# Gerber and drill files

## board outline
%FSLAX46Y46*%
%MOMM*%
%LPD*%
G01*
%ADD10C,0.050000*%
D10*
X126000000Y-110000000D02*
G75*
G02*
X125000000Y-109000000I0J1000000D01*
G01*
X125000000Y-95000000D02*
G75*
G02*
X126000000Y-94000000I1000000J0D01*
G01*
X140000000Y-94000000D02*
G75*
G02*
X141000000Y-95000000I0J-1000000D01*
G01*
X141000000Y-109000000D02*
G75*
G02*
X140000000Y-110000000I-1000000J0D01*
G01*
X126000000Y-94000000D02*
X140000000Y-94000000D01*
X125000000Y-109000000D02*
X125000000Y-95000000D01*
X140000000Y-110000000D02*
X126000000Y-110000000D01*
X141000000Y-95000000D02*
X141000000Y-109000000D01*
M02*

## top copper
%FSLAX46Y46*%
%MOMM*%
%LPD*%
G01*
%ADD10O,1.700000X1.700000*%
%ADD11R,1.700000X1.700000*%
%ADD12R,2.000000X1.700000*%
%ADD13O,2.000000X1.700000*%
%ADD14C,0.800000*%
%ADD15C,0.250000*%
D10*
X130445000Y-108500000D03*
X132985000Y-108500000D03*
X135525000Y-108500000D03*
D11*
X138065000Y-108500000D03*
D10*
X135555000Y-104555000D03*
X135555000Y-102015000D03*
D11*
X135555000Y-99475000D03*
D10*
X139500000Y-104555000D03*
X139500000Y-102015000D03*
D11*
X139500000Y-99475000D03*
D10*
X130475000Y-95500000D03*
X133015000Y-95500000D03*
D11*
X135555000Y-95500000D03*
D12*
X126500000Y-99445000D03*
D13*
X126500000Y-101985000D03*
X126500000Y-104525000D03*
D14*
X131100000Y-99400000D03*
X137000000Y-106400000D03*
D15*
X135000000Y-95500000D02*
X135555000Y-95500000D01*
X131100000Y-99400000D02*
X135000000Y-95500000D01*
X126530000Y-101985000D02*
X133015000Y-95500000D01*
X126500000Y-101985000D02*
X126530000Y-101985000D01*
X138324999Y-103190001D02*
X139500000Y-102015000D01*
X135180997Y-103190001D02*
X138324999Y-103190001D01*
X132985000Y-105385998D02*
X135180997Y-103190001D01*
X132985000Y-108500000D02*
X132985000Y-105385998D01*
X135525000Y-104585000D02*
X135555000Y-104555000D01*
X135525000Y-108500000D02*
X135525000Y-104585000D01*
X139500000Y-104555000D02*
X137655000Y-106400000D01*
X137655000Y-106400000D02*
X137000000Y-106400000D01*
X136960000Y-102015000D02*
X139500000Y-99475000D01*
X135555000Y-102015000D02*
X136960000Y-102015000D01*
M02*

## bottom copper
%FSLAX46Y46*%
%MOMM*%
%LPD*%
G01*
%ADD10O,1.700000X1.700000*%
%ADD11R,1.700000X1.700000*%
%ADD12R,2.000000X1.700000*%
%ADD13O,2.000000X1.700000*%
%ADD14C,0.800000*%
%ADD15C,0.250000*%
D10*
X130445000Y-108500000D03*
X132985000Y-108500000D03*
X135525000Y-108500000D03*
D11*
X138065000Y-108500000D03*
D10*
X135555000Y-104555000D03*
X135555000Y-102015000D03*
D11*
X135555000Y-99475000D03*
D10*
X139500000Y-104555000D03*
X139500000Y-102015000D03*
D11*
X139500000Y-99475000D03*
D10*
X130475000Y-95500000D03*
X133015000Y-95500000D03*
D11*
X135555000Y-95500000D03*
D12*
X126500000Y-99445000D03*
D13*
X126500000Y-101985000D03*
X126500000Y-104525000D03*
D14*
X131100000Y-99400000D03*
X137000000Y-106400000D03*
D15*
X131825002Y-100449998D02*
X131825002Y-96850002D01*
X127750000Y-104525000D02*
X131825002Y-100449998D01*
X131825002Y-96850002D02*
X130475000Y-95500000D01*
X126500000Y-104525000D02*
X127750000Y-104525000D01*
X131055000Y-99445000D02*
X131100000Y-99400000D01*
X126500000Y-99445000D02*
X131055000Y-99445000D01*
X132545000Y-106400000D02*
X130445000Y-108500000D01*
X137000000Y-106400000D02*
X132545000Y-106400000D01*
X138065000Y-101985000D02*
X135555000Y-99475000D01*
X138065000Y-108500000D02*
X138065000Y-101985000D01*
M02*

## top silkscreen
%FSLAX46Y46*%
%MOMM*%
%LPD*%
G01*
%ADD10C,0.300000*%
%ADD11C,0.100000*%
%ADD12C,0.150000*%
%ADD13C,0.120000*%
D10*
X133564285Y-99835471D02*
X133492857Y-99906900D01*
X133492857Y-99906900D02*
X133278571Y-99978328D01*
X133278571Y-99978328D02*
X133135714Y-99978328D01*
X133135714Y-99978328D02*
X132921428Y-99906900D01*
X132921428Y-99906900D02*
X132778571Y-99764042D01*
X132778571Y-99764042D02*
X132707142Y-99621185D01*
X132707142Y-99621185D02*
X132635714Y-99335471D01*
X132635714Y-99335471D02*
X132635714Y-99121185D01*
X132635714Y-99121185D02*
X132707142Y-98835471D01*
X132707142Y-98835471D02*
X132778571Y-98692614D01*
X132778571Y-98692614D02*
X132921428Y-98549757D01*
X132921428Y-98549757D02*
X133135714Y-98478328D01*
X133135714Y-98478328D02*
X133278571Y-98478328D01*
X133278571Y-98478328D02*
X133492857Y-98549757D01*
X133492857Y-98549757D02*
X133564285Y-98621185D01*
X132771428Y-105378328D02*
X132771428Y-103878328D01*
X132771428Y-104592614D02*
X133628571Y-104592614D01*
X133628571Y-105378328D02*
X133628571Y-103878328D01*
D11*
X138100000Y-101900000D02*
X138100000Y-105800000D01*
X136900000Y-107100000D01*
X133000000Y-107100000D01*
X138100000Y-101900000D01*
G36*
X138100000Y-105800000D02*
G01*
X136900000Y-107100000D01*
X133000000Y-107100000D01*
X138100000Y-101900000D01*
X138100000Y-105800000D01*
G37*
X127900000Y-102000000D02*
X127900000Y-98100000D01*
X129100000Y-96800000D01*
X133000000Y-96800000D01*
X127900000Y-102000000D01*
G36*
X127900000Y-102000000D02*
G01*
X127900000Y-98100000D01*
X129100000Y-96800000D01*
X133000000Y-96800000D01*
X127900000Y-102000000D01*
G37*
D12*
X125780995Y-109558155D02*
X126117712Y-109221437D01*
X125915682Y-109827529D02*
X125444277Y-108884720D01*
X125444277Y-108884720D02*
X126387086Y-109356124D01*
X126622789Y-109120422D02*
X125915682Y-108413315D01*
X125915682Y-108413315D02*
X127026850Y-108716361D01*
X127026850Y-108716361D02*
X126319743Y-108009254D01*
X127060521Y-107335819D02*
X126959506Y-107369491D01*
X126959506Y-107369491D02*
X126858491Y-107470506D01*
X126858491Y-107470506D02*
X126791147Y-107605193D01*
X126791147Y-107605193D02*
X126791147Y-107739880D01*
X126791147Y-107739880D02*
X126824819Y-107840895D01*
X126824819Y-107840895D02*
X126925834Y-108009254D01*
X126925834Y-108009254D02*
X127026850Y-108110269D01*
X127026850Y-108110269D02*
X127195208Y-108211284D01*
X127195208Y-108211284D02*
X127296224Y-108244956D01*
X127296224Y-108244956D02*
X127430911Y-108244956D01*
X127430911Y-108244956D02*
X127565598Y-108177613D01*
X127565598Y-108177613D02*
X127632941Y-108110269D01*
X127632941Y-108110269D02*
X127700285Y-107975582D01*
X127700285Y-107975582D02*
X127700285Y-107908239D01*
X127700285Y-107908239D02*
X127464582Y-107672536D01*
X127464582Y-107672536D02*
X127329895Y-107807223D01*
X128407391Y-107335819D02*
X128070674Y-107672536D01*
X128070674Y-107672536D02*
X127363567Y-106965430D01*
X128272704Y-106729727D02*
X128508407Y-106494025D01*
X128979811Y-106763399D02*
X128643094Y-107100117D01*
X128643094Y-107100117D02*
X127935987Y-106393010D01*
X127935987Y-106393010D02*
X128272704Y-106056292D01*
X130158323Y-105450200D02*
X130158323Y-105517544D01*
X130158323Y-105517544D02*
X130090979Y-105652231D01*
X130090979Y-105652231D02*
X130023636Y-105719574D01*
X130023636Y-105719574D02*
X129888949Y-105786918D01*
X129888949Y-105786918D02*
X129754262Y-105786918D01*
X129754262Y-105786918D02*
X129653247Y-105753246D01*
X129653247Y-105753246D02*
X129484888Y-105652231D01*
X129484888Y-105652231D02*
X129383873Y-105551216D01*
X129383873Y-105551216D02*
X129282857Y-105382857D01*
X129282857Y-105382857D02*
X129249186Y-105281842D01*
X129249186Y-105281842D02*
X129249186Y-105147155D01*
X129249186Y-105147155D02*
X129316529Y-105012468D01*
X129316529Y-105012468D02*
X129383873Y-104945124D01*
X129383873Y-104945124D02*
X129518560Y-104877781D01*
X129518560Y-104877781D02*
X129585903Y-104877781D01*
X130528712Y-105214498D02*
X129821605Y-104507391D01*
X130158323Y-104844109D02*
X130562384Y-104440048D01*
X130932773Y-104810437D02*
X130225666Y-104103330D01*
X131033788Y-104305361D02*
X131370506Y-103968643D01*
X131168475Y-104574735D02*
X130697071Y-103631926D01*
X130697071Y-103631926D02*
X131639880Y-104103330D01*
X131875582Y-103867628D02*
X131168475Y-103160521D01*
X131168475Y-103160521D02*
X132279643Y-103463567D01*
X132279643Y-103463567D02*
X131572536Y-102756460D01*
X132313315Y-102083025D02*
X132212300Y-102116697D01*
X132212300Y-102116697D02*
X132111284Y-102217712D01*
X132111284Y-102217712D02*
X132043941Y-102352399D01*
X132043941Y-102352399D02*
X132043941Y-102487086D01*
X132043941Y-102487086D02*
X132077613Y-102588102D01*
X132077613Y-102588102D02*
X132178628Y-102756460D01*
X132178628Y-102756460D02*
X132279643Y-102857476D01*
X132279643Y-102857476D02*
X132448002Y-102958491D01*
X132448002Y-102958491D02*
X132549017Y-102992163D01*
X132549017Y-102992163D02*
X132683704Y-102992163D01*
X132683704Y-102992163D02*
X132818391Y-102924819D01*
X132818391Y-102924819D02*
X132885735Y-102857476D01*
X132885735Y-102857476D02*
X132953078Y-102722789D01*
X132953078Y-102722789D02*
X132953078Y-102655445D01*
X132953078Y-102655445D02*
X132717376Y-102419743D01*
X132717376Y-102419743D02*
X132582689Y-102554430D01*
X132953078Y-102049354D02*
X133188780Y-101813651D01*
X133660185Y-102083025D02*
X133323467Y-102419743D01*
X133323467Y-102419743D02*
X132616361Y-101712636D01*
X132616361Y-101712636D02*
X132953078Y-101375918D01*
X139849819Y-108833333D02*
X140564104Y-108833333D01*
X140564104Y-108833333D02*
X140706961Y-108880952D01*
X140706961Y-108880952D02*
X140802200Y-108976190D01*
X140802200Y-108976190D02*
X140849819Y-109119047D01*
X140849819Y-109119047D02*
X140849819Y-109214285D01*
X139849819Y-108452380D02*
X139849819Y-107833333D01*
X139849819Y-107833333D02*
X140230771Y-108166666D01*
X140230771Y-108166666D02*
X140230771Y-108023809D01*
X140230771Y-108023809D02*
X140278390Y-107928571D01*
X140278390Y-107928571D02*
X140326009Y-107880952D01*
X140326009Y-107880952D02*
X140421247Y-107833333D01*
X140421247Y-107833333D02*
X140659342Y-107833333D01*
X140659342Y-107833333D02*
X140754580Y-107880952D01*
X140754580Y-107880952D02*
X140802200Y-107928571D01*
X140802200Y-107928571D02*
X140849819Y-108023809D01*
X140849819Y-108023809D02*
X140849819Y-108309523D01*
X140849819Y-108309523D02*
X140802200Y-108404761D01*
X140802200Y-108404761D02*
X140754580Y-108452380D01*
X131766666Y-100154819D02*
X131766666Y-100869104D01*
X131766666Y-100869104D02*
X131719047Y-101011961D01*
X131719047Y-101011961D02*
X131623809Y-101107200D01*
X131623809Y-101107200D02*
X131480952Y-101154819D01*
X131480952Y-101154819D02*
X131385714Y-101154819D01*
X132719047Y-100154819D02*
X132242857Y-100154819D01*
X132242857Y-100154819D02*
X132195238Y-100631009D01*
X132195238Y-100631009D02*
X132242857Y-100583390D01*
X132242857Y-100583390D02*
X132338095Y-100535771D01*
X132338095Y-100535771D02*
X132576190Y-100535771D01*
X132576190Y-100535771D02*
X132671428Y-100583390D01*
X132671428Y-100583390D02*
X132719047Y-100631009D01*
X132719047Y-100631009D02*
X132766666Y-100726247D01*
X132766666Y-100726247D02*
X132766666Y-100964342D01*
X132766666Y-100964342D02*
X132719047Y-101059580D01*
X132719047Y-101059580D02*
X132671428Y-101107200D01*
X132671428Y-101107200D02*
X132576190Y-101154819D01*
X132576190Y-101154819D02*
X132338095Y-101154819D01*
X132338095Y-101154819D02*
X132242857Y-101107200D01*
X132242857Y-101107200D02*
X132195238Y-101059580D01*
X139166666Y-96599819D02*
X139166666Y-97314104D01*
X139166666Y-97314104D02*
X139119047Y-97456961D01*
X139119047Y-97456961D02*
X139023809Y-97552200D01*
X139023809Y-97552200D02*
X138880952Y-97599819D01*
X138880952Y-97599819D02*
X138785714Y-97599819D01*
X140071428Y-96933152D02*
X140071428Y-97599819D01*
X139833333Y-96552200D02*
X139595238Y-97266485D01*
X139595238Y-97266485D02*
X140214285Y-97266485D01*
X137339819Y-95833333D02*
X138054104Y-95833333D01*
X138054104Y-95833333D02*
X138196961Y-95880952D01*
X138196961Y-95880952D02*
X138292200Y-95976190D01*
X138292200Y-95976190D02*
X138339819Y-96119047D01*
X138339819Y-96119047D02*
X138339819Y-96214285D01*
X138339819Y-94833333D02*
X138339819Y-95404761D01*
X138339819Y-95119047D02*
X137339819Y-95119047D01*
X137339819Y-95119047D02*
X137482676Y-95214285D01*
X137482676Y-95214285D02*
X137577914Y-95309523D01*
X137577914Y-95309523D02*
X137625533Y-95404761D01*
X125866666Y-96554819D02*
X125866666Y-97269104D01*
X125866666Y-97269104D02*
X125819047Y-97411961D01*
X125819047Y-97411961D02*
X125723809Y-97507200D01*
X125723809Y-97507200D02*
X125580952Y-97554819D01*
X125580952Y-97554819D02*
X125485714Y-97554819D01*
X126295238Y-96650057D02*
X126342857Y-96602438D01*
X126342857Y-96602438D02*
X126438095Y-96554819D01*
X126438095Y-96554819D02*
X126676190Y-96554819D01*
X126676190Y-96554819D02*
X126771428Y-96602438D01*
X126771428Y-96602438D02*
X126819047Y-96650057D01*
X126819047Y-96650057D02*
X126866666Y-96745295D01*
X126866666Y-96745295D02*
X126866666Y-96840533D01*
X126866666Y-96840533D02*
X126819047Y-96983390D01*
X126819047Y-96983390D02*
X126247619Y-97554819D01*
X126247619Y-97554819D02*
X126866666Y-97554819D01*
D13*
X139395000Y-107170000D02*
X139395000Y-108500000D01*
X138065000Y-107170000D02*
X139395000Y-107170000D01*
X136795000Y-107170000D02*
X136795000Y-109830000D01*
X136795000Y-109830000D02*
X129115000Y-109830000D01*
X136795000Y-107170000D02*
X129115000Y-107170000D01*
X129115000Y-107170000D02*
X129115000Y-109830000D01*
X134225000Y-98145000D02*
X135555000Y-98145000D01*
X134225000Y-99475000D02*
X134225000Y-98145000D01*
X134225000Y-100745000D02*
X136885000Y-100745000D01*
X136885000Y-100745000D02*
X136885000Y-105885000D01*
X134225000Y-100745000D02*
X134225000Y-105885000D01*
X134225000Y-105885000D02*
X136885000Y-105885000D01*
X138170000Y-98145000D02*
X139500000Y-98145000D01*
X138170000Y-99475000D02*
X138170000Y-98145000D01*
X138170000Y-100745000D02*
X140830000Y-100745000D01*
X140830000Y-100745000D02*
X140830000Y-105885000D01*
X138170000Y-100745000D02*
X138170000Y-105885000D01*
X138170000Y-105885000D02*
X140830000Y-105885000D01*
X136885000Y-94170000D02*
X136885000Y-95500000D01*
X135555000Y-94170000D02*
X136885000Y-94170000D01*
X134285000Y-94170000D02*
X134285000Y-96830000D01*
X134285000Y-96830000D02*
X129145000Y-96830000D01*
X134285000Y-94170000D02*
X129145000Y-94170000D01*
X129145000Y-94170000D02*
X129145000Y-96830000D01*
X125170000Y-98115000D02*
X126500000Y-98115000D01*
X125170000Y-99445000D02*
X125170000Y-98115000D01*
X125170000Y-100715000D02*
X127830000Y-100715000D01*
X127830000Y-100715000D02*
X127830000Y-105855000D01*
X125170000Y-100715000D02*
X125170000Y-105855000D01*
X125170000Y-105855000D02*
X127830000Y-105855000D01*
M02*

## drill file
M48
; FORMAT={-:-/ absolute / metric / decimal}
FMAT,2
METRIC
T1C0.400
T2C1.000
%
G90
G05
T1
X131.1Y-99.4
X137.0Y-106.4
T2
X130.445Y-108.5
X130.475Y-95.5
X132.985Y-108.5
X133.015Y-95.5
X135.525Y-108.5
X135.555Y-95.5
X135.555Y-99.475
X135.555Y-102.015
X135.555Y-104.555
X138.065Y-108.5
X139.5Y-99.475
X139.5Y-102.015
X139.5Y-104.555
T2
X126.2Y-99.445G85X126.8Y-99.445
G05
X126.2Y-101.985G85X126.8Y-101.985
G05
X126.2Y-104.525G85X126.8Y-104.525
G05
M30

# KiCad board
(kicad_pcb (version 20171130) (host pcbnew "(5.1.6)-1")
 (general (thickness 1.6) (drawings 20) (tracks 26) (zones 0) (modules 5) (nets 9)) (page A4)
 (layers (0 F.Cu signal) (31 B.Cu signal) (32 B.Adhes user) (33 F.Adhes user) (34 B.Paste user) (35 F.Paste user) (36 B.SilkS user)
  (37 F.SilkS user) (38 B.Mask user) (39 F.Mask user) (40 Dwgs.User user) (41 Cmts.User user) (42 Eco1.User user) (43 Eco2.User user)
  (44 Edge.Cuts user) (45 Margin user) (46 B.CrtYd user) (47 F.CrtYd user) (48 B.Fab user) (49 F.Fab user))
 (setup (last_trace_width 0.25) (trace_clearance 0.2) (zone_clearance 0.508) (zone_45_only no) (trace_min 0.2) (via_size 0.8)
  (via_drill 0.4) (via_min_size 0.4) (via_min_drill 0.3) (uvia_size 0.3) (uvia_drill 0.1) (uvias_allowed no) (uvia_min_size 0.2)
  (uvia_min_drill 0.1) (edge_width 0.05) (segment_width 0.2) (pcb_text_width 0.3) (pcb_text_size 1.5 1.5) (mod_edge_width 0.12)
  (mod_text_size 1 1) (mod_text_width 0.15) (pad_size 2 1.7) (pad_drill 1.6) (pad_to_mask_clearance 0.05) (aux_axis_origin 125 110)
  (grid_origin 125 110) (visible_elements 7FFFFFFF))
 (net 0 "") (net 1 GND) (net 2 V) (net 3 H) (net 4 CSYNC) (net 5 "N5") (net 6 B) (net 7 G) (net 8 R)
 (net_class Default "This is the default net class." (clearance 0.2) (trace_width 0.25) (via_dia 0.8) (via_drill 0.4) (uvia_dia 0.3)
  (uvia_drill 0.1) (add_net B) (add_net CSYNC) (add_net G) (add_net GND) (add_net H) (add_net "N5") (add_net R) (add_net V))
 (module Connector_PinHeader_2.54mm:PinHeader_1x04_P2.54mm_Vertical (layer F.Cu) (at 138.065 108.5 270)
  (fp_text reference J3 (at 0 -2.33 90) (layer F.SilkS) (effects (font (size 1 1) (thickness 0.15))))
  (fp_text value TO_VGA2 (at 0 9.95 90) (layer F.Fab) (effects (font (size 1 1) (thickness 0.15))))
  (fp_line (start -1.33 -1.33) (end 0 -1.33) (layer F.SilkS) (width 0.12))
  (fp_line (start -1.33 0) (end -1.33 -1.33) (layer F.SilkS) (width 0.12))
  (fp_line (start -1.33 1.27) (end 1.33 1.27) (layer F.SilkS) (width 0.12))
  (fp_line (start 1.33 1.27) (end 1.33 8.95) (layer F.SilkS) (width 0.12))
  (fp_line (start -1.33 1.27) (end -1.33 8.95) (layer F.SilkS) (width 0.12))
  (fp_line (start -1.33 8.95) (end 1.33 8.95) (layer F.SilkS) (width 0.12))
  (pad 4 thru_hole oval (at 0 7.62 270) (size 1.7 1.7) (drill 1) (layers *.Cu *.Mask) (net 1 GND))
  (pad 3 thru_hole oval (at 0 5.08 270) (size 1.7 1.7) (drill 1) (layers *.Cu *.Mask) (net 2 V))
  (pad 2 thru_hole oval (at 0 2.54 270) (size 1.7 1.7) (drill 1) (layers *.Cu *.Mask) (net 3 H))
  (pad 1 thru_hole rect (at 0 0 270) (size 1.7 1.7) (drill 1) (layers *.Cu *.Mask) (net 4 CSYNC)))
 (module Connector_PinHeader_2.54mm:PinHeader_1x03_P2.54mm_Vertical (layer F.Cu) (at 135.555 99.475)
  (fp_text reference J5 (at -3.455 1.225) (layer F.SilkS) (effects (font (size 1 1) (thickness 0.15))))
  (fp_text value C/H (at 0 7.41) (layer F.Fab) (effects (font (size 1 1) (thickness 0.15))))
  (fp_line (start -1.33 -1.33) (end 0 -1.33) (layer F.SilkS) (width 0.12))
  (fp_line (start -1.33 0) (end -1.33 -1.33) (layer F.SilkS) (width 0.12))
  (fp_line (start -1.33 1.27) (end 1.33 1.27) (layer F.SilkS) (width 0.12))
  (fp_line (start 1.33 1.27) (end 1.33 6.41) (layer F.SilkS) (width 0.12))
  (fp_line (start -1.33 1.27) (end -1.33 6.41) (layer F.SilkS) (width 0.12))
  (fp_line (start -1.33 6.41) (end 1.33 6.41) (layer F.SilkS) (width 0.12))
  (pad 3 thru_hole oval (at 0 5.08) (size 1.7 1.7) (drill 1) (layers *.Cu *.Mask) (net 3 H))
  (pad 2 thru_hole oval (at 0 2.54) (size 1.7 1.7) (drill 1) (layers *.Cu *.Mask) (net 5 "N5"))
  (pad 1 thru_hole rect (at 0 0) (size 1.7 1.7) (drill 1) (layers *.Cu *.Mask) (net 4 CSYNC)))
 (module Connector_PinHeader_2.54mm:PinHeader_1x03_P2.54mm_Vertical (layer F.Cu) (at 139.5 99.475)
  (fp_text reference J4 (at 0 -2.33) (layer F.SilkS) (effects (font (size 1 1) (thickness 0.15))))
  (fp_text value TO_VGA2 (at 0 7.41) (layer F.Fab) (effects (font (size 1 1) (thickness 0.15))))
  (fp_line (start -1.33 -1.33) (end 0 -1.33) (layer F.SilkS) (width 0.12))
  (fp_line (start -1.33 0) (end -1.33 -1.33) (layer F.SilkS) (width 0.12))
  (fp_line (start -1.33 1.27) (end 1.33 1.27) (layer F.SilkS) (width 0.12))
  (fp_line (start 1.33 1.27) (end 1.33 6.41) (layer F.SilkS) (width 0.12))
  (fp_line (start -1.33 1.27) (end -1.33 6.41) (layer F.SilkS) (width 0.12))
  (fp_line (start -1.33 6.41) (end 1.33 6.41) (layer F.SilkS) (width 0.12))
  (pad 3 thru_hole oval (at 0 5.08) (size 1.7 1.7) (drill 1) (layers *.Cu *.Mask) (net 1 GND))
  (pad 2 thru_hole oval (at 0 2.54) (size 1.7 1.7) (drill 1) (layers *.Cu *.Mask) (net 2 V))
  (pad 1 thru_hole rect (at 0 0) (size 1.7 1.7) (drill 1) (layers *.Cu *.Mask) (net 5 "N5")))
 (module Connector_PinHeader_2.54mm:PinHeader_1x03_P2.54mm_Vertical (layer F.Cu) (at 135.555 95.5 270)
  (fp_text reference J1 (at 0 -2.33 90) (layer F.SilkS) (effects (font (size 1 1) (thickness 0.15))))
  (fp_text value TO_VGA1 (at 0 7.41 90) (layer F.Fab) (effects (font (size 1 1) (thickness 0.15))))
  (fp_line (start -1.33 -1.33) (end 0 -1.33) (layer F.SilkS) (width 0.12))
  (fp_line (start -1.33 0) (end -1.33 -1.33) (layer F.SilkS) (width 0.12))
  (fp_line (start -1.33 1.27) (end 1.33 1.27) (layer F.SilkS) (width 0.12))
  (fp_line (start 1.33 1.27) (end 1.33 6.41) (layer F.SilkS) (width 0.12))
  (fp_line (start -1.33 1.27) (end -1.33 6.41) (layer F.SilkS) (width 0.12))
  (fp_line (start -1.33 6.41) (end 1.33 6.41) (layer F.SilkS) (width 0.12))
  (pad 3 thru_hole oval (at 0 5.08 270) (size 1.7 1.7) (drill 1) (layers *.Cu *.Mask) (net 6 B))
  (pad 2 thru_hole oval (at 0 2.54 270) (size 1.7 1.7) (drill 1) (layers *.Cu *.Mask) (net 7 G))
  (pad 1 thru_hole rect (at 0 0 270) (size 1.7 1.7) (drill 1) (layers *.Cu *.Mask) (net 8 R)))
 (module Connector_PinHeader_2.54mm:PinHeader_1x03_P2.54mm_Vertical (layer F.Cu) (at 126.5 99.445)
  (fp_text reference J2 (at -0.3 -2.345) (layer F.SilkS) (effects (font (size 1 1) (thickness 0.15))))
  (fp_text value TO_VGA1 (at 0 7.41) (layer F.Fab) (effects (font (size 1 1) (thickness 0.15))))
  (fp_line (start -1.33 -1.33) (end 0 -1.33) (layer F.SilkS) (width 0.12))
  (fp_line (start -1.33 0) (end -1.33 -1.33) (layer F.SilkS) (width 0.12))
  (fp_line (start -1.33 1.27) (end 1.33 1.27) (layer F.SilkS) (width 0.12))
  (fp_line (start 1.33 1.27) (end 1.33 6.41) (layer F.SilkS) (width 0.12))
  (fp_line (start -1.33 1.27) (end -1.33 6.41) (layer F.SilkS) (width 0.12))
  (fp_line (start -1.33 6.41) (end 1.33 6.41) (layer F.SilkS) (width 0.12))
  (pad 1 thru_hole rect (at 0 0) (size 2 1.7) (drill oval 1.6 1) (layers *.Cu *.Mask) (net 8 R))
  (pad 2 thru_hole oval (at 0 2.54) (size 2 1.7) (drill oval 1.6 1) (layers *.Cu *.Mask) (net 7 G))
  (pad 3 thru_hole oval (at 0 5.08) (size 2 1.7) (drill oval 1.6 1) (layers *.Cu *.Mask) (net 6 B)))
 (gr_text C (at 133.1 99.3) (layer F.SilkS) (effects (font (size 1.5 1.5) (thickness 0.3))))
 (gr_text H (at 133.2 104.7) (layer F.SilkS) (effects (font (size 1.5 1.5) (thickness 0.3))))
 (gr_poly (pts (xy 138.1 101.9) (xy 138.1 105.8) (xy 136.9 107.1) (xy 133 107.1)) (layer F.SilkS) (width 0.1))
 (gr_poly (pts (xy 127.9 102) (xy 127.9 98.1) (xy 129.1 96.8) (xy 133 96.8)) (layer F.SilkS) (width 0.1))
 (gr_arc (start 126 109) (end 125 109) (angle -90) (layer Edge.Cuts) (width 0.05))
 (gr_arc (start 126 95) (end 126 94) (angle -90) (layer Edge.Cuts) (width 0.05))
 (gr_arc (start 140 95) (end 141 95) (angle -90) (layer Edge.Cuts) (width 0.05))
 (gr_arc (start 140 109) (end 140 110) (angle -90) (layer Edge.Cuts) (width 0.05))
 (gr_line (start 126 94) (end 140 94) (layer Edge.Cuts) (width 0.05))
 (gr_line (start 125 109) (end 125 95) (layer Edge.Cuts) (width 0.05))
 (gr_line (start 140 110) (end 126 110) (layer Edge.Cuts) (width 0.05))
 (gr_line (start 141 95) (end 141 109) (layer Edge.Cuts) (width 0.05))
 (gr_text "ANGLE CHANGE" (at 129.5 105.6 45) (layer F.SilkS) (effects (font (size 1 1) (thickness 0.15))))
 (segment (start 131.825002 100.449998) (end 131.825002 96.850002) (width 0.25) (layer B.Cu) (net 6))
 (segment (start 127.75 104.525) (end 131.825002 100.449998) (width 0.25) (layer B.Cu) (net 6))
 (segment (start 131.825002 96.850002) (end 130.475 95.5) (width 0.25) (layer B.Cu) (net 6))
 (segment (start 126.5 104.525) (end 127.75 104.525) (width 0.25) (layer B.Cu) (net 6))
 (via (at 131.1 99.4) (size 0.8) (drill 0.4) (layers F.Cu B.Cu) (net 8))
 (segment (start 131.055 99.445) (end 131.1 99.4) (width 0.25) (layer B.Cu) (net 8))
 (segment (start 126.5 99.445) (end 131.055 99.445) (width 0.25) (layer B.Cu) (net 8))
 (segment (start 135 95.5) (end 135.555 95.5) (width 0.25) (layer F.Cu) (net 8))
 (segment (start 131.1 99.4) (end 135 95.5) (width 0.25) (layer F.Cu) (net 8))
 (segment (start 126.53 101.985) (end 133.015 95.5) (width 0.25) (layer F.Cu) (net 7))
 (segment (start 126.5 101.985) (end 126.53 101.985) (width 0.25) (layer F.Cu) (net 7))
 (segment (start 138.324999 103.190001) (end 139.5 102.015) (width 0.25) (layer F.Cu) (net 2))
 (segment (start 135.180997 103.190001) (end 138.324999 103.190001) (width 0.25) (layer F.Cu) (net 2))
 (segment (start 132.985 105.385998) (end 135.180997 103.190001) (width 0.25) (layer F.Cu) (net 2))
 (segment (start 132.985 108.5) (end 132.985 105.385998) (width 0.25) (layer F.Cu) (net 2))
 (segment (start 135.525 104.585) (end 135.555 104.555) (width 0.25) (layer F.Cu) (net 3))
 (segment (start 135.525 108.5) (end 135.525 104.585) (width 0.25) (layer F.Cu) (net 3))
 (via (at 137 106.4) (size 0.8) (drill 0.4) (layers F.Cu B.Cu) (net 1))
 (segment (start 139.5 104.555) (end 137.655 106.4) (width 0.25) (layer F.Cu) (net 1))
 (segment (start 137.655 106.4) (end 137 106.4) (width 0.25) (layer F.Cu) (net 1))
 (segment (start 132.545 106.4) (end 130.445 108.5) (width 0.25) (layer B.Cu) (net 1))
 (segment (start 137 106.4) (end 132.545 106.4) (width 0.25) (layer B.Cu) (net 1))
 (segment (start 138.065 101.985) (end 135.555 99.475) (width 0.25) (layer B.Cu) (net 4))
 (segment (start 138.065 108.5) (end 138.065 101.985) (width 0.25) (layer B.Cu) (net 4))
 (segment (start 136.96 102.015) (end 139.5 99.475) (width 0.25) (layer F.Cu) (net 5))
 (segment (start 135.555 102.015) (end 136.96 102.015) (width 0.25) (layer F.Cu) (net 5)))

